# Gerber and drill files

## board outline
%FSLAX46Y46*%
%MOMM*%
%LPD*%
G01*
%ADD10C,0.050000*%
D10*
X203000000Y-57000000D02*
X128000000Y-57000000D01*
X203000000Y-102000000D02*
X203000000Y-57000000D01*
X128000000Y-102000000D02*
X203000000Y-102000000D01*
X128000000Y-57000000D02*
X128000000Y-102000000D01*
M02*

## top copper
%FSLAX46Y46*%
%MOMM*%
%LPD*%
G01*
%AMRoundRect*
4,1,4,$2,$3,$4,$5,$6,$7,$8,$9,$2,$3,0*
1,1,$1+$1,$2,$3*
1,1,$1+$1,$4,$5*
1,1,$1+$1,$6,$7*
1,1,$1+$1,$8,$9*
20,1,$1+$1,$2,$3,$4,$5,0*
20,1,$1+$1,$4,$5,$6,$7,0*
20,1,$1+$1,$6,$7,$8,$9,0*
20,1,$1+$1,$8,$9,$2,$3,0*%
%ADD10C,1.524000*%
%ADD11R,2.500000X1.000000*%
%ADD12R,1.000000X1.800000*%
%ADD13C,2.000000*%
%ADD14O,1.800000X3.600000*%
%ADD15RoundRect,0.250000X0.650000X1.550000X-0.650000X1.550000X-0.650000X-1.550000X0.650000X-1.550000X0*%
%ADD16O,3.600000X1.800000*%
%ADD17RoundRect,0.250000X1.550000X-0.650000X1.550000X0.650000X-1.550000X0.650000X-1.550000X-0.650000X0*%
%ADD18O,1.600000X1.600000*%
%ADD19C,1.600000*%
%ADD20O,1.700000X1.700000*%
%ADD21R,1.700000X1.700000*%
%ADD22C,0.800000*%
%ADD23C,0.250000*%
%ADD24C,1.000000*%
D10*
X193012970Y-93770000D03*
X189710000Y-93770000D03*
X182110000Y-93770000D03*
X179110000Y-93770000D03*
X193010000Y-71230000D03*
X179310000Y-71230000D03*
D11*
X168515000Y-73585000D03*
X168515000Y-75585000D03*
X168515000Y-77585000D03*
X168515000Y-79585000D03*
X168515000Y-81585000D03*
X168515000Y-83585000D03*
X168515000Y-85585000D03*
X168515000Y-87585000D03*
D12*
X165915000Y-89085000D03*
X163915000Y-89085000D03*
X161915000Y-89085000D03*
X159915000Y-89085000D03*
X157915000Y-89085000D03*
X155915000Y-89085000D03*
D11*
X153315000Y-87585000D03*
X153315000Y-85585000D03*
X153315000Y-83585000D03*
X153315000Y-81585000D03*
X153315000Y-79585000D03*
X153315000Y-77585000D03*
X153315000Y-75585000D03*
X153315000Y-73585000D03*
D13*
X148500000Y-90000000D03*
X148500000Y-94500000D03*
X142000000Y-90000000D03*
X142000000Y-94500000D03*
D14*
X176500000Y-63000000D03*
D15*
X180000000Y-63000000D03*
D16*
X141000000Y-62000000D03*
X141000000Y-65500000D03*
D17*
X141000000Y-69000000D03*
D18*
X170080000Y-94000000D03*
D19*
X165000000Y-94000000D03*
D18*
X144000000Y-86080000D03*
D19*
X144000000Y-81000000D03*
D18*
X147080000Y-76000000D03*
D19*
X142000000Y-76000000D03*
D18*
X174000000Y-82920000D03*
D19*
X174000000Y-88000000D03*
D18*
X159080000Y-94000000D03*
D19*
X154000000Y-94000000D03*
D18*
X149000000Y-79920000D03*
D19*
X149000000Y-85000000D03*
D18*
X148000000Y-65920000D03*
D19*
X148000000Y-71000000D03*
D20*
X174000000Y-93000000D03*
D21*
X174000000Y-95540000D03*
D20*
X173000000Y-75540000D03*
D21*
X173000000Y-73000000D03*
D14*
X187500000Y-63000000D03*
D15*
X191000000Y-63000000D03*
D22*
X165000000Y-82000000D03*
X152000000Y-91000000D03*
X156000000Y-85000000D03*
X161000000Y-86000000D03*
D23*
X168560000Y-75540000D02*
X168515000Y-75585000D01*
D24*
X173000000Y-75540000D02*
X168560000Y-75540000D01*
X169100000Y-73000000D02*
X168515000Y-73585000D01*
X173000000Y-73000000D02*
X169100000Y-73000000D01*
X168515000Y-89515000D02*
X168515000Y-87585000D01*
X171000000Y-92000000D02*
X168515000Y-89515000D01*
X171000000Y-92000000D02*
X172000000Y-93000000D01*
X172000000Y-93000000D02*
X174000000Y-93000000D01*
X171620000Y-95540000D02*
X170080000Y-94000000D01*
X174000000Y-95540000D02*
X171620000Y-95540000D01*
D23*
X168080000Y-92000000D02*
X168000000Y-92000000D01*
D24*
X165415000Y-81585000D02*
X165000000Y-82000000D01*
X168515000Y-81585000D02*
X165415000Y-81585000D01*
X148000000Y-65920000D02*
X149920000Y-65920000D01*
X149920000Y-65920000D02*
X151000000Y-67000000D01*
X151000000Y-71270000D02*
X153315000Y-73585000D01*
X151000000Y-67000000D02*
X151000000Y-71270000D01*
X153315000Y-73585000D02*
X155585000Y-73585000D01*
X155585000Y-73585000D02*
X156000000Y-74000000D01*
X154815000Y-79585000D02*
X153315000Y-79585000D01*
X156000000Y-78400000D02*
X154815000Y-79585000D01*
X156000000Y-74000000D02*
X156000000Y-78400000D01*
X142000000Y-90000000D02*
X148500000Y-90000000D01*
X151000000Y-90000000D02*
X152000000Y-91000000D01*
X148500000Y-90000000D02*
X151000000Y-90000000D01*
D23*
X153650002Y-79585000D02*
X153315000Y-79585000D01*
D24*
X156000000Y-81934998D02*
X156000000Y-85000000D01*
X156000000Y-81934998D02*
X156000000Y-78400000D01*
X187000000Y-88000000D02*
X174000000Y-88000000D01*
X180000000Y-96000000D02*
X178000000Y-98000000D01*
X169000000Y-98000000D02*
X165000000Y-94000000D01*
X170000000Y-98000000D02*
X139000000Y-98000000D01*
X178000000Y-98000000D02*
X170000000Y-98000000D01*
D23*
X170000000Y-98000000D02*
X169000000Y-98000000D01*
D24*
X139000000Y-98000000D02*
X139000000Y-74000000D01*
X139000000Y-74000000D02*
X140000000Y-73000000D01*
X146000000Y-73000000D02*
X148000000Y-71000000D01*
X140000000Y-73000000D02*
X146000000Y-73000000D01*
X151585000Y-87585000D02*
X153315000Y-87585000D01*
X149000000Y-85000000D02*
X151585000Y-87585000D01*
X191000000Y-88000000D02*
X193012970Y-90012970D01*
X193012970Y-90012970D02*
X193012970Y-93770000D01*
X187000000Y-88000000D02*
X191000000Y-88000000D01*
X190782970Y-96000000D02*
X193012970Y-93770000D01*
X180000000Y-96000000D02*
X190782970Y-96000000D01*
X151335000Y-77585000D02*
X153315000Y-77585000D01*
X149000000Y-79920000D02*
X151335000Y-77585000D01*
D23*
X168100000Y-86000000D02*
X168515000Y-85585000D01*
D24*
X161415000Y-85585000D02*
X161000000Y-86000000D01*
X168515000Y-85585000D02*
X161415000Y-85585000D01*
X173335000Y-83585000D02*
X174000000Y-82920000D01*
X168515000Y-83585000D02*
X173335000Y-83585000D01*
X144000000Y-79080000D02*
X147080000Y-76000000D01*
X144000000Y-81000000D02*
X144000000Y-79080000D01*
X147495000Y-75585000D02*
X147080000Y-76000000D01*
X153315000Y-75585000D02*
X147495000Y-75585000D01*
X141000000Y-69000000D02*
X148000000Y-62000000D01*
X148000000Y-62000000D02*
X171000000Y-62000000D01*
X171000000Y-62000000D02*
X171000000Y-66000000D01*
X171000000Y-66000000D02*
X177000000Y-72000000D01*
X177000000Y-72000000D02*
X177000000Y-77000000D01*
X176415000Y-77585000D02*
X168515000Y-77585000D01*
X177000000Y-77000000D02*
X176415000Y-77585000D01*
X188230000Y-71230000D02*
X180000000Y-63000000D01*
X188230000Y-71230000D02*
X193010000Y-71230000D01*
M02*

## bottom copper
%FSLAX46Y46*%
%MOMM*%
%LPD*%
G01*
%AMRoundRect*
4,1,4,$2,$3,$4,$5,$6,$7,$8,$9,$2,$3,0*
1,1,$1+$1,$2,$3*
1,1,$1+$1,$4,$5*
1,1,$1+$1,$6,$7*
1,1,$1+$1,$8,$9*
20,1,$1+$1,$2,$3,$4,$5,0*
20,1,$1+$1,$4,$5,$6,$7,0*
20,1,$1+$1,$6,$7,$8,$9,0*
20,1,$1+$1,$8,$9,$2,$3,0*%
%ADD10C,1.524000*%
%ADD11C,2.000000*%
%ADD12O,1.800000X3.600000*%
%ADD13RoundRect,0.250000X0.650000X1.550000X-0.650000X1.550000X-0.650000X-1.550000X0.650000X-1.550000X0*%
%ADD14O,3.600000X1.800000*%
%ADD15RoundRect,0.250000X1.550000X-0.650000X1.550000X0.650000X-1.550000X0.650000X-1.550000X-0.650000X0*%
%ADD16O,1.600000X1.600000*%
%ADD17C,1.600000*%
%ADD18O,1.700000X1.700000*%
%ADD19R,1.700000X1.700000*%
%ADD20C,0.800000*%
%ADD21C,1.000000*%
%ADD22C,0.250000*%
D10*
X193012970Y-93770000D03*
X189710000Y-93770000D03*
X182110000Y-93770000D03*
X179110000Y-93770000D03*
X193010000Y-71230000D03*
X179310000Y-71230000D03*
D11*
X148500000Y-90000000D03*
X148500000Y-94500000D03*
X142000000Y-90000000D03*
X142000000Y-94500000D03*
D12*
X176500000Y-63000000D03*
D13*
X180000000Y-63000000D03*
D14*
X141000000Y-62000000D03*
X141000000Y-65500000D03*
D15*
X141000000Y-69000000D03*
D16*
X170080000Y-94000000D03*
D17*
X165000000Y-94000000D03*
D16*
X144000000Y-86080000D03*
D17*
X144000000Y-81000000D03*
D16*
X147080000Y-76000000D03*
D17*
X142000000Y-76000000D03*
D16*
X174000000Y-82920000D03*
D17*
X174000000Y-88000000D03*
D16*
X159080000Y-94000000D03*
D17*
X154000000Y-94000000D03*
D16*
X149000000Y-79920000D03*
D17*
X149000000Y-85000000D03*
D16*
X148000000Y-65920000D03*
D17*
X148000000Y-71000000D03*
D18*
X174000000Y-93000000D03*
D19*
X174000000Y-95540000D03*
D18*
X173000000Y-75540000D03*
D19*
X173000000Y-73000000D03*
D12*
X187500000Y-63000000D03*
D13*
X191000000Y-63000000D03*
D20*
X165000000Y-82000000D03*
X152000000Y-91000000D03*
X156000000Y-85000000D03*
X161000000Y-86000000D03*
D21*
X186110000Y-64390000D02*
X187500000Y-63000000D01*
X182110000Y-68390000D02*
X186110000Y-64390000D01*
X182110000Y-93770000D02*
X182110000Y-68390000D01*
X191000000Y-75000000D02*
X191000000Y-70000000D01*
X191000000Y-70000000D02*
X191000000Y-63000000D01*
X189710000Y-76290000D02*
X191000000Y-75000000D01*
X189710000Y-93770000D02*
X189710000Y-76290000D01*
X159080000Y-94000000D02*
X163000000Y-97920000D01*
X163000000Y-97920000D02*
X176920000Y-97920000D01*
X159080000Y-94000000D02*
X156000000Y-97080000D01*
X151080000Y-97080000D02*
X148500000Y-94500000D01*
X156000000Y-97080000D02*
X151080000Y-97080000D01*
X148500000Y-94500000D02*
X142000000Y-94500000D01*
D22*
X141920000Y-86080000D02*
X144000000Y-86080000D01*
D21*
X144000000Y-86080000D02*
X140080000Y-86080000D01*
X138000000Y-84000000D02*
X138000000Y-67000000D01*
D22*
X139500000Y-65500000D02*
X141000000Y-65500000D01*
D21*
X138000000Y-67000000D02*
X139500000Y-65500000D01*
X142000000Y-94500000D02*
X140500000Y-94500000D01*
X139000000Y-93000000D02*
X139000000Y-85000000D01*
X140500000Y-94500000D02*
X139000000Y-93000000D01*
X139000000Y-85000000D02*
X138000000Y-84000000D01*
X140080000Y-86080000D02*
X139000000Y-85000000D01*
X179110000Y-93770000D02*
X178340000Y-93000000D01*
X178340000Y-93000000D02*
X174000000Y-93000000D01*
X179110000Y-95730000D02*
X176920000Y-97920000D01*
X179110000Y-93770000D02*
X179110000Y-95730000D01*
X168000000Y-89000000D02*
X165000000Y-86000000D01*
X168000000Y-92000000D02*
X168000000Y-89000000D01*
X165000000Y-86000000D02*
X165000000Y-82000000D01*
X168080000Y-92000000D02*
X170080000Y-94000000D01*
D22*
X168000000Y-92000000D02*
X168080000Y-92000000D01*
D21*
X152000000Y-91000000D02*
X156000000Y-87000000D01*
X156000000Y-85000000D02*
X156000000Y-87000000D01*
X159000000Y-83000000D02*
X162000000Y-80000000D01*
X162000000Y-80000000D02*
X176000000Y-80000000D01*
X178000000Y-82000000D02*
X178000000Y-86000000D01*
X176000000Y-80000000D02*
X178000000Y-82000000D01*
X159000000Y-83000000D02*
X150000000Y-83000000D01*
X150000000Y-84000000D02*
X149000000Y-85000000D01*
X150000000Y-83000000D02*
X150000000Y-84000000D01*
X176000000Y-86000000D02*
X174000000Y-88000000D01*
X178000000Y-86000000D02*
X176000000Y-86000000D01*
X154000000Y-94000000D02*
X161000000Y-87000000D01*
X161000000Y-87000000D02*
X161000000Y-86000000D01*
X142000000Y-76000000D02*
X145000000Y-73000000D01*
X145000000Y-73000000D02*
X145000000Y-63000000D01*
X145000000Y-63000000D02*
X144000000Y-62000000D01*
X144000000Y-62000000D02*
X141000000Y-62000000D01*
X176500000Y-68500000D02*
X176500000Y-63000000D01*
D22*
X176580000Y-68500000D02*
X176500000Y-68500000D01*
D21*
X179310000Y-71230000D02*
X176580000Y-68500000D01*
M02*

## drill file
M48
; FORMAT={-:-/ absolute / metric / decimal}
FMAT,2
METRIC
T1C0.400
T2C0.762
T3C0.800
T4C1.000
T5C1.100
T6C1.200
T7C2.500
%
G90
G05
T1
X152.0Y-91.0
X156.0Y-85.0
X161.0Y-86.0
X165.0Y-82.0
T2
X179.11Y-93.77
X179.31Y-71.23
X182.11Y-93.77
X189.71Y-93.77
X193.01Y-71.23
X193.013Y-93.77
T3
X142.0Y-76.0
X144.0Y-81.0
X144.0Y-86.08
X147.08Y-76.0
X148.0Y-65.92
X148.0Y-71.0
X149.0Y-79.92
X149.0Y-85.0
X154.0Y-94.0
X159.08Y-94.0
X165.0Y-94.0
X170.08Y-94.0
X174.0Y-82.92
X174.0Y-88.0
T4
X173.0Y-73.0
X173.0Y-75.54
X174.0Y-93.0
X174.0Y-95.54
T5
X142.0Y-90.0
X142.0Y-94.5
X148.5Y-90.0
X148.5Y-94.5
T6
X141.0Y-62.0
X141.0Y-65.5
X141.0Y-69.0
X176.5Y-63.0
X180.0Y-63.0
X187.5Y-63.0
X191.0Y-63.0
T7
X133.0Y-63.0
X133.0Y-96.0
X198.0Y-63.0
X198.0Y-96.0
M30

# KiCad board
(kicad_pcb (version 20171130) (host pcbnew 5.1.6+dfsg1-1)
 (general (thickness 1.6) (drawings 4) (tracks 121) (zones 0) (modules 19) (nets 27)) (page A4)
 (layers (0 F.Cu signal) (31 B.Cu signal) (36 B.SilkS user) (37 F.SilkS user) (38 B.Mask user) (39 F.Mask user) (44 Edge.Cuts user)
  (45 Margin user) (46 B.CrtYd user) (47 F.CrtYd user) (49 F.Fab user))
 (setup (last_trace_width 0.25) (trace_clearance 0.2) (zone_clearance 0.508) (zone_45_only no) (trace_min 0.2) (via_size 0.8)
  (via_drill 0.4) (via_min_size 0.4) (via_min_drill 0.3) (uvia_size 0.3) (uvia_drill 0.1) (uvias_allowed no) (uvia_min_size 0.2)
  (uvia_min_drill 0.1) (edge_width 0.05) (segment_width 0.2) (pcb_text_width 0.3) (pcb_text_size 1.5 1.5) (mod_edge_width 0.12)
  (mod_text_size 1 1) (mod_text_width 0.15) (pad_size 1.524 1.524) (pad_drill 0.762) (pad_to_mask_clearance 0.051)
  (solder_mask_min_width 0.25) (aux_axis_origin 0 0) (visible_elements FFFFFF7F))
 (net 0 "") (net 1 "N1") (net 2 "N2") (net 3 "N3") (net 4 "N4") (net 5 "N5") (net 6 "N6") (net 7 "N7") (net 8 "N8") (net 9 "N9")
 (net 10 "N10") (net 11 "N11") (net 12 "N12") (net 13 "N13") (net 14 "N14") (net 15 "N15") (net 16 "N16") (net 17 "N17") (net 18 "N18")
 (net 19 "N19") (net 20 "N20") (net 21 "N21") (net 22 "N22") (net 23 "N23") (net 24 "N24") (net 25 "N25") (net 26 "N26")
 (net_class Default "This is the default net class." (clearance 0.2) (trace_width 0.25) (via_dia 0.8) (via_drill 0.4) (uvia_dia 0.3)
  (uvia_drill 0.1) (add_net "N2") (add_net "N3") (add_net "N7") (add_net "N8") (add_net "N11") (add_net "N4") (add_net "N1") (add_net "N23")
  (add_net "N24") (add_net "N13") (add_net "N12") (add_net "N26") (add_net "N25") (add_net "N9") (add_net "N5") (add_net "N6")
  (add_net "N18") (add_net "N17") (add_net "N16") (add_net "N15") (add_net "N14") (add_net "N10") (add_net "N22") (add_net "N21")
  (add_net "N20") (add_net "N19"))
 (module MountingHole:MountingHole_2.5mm (layer F.Cu) (at 133 63)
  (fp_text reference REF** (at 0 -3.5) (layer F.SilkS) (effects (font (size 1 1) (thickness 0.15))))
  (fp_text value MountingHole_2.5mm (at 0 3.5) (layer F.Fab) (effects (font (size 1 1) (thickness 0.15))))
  (pad 1 np_thru_hole circle (at 0 0) (size 2.5 2.5) (drill 2.5) (layers *.Cu *.Mask)))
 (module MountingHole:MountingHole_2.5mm (layer F.Cu) (at 133 96)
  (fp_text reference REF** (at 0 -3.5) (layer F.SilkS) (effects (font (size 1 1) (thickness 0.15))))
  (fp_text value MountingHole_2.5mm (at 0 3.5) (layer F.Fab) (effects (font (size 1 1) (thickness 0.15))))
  (pad 1 np_thru_hole circle (at 0 0) (size 2.5 2.5) (drill 2.5) (layers *.Cu *.Mask)))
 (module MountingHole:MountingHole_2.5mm (layer F.Cu) (at 198 96)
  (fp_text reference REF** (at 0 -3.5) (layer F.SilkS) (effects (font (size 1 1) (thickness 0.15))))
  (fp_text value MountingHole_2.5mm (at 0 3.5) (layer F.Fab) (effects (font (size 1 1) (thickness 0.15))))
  (pad 1 np_thru_hole circle (at 0 0) (size 2.5 2.5) (drill 2.5) (layers *.Cu *.Mask)))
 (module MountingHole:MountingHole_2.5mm (layer F.Cu) (at 198 63)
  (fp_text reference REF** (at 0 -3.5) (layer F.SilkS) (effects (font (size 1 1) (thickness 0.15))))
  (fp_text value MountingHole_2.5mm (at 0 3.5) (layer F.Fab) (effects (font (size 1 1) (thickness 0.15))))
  (pad 1 np_thru_hole circle (at 0 0) (size 2.5 2.5) (drill 2.5) (layers *.Cu *.Mask)))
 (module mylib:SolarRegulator (layer F.Cu) (at 186 83)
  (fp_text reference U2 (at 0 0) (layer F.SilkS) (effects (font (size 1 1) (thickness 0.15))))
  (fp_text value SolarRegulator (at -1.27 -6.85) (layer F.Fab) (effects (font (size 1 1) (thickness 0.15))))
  (pad 6 thru_hole circle (at 7.01297 10.77) (size 1.524 1.524) (drill 0.762) (layers *.Cu *.Mask) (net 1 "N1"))
  (pad 5 thru_hole circle (at 3.71 10.77) (size 1.524 1.524) (drill 0.762) (layers *.Cu *.Mask) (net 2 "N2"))
  (pad 4 thru_hole circle (at -3.89 10.77) (size 1.524 1.524) (drill 0.762) (layers *.Cu *.Mask) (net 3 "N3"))
  (pad 3 thru_hole circle (at -6.89 10.77) (size 1.524 1.524) (drill 0.762) (layers *.Cu *.Mask) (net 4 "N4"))
  (pad 2 thru_hole circle (at 7.01 -11.77) (size 1.524 1.524) (drill 0.762) (layers *.Cu *.Mask) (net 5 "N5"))
  (pad 1 thru_hole circle (at -6.69 -11.77) (size 1.524 1.524) (drill 0.762) (layers *.Cu *.Mask) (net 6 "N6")))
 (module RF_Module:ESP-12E (layer F.Cu) (at 160.915 77.085)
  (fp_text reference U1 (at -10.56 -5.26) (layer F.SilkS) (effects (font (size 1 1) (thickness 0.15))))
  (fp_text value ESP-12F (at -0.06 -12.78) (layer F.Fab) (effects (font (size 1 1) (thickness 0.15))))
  (pad 22 smd rect (at 7.6 -3.5) (size 2.5 1) (layers F.Cu F.Paste F.Mask) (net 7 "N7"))
  (pad 21 smd rect (at 7.6 -1.5) (size 2.5 1) (layers F.Cu F.Paste F.Mask) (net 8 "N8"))
  (pad 20 smd rect (at 7.6 0.5) (size 2.5 1) (layers F.Cu F.Paste F.Mask) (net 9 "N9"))
  (pad 19 smd rect (at 7.6 2.5) (size 2.5 1) (layers F.Cu F.Paste F.Mask) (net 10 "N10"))
  (pad 18 smd rect (at 7.6 4.5) (size 2.5 1) (layers F.Cu F.Paste F.Mask) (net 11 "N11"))
  (pad 17 smd rect (at 7.6 6.5) (size 2.5 1) (layers F.Cu F.Paste F.Mask) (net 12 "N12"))
  (pad 16 smd rect (at 7.6 8.5) (size 2.5 1) (layers F.Cu F.Paste F.Mask) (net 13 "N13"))
  (pad 15 smd rect (at 7.6 10.5) (size 2.5 1) (layers F.Cu F.Paste F.Mask) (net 4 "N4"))
  (pad 14 smd rect (at 5 12) (size 1 1.8) (layers F.Cu F.Paste F.Mask) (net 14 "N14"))
  (pad 13 smd rect (at 3 12) (size 1 1.8) (layers F.Cu F.Paste F.Mask) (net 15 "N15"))
  (pad 12 smd rect (at 1 12) (size 1 1.8) (layers F.Cu F.Paste F.Mask) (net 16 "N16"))
  (pad 11 smd rect (at -1 12) (size 1 1.8) (layers F.Cu F.Paste F.Mask) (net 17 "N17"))
  (pad 10 smd rect (at -3 12) (size 1 1.8) (layers F.Cu F.Paste F.Mask) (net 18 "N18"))
  (pad 9 smd rect (at -5 12) (size 1 1.8) (layers F.Cu F.Paste F.Mask) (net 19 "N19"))
  (pad 8 smd rect (at -7.6 10.5) (size 2.5 1) (layers F.Cu F.Paste F.Mask) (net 1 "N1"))
  (pad 7 smd rect (at -7.6 8.5) (size 2.5 1) (layers F.Cu F.Paste F.Mask) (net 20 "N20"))
  (pad 6 smd rect (at -7.6 6.5) (size 2.5 1) (layers F.Cu F.Paste F.Mask) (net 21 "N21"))
  (pad 5 smd rect (at -7.6 4.5) (size 2.5 1) (layers F.Cu F.Paste F.Mask) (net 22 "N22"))
  (pad 4 smd rect (at -7.6 2.5) (size 2.5 1) (layers F.Cu F.Paste F.Mask) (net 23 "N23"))
  (pad 3 smd rect (at -7.6 0.5) (size 2.5 1) (layers F.Cu F.Paste F.Mask) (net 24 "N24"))
  (pad 2 smd rect (at -7.6 -1.5) (size 2.5 1) (layers F.Cu F.Paste F.Mask) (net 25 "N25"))
  (pad 1 smd rect (at -7.6 -3.5) (size 2.5 1) (layers F.Cu F.Paste F.Mask) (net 23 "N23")))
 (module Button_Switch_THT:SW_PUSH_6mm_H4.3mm (layer F.Cu) (at 142 90)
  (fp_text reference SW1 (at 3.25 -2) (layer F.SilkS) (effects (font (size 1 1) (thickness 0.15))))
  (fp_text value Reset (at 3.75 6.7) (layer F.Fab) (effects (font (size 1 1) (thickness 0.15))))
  (pad 1 thru_hole circle (at 6.5 0 90) (size 2 2) (drill 1.1) (layers *.Cu *.Mask) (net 23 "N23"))
  (pad 2 thru_hole circle (at 6.5 4.5 90) (size 2 2) (drill 1.1) (layers *.Cu *.Mask) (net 4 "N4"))
  (pad 1 thru_hole circle (at 0 0 90) (size 2 2) (drill 1.1) (layers *.Cu *.Mask) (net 23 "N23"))
  (pad 2 thru_hole circle (at 0 4.5 90) (size 2 2) (drill 1.1) (layers *.Cu *.Mask) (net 4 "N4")))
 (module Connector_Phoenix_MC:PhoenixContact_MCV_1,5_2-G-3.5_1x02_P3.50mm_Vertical (layer F.Cu) (at 180 63 180)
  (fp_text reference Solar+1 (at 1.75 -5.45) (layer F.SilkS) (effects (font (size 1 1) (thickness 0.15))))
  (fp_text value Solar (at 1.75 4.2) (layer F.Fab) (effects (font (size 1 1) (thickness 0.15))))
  (pad 2 thru_hole oval (at 3.5 0 180) (size 1.8 3.6) (drill 1.2) (layers *.Cu *.Mask) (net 6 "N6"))
  (pad 1 thru_hole roundrect (at 0 0 180) (size 1.8 3.6) (drill 1.2) (layers *.Cu *.Mask) (roundrect_rratio 0.138889) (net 5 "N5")))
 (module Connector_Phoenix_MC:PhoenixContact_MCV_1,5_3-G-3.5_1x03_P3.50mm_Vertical (layer F.Cu) (at 141 69 90)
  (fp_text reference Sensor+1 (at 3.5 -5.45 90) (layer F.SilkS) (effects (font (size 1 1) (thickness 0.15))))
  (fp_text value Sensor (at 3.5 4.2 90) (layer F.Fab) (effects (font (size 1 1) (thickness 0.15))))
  (pad 3 thru_hole oval (at 7 0 90) (size 1.8 3.6) (drill 1.2) (layers *.Cu *.Mask) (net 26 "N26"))
  (pad 2 thru_hole oval (at 3.5 0 90) (size 1.8 3.6) (drill 1.2) (layers *.Cu *.Mask) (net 4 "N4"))
  (pad 1 thru_hole roundrect (at 0 0 90) (size 1.8 3.6) (drill 1.2) (layers *.Cu *.Mask) (roundrect_rratio 0.138889) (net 9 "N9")))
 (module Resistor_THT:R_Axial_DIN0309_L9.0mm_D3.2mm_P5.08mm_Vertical (layer F.Cu) (at 165 94)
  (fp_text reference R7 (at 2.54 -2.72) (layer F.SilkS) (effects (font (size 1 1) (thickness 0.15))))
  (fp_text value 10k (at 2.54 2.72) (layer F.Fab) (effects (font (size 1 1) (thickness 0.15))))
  (pad 2 thru_hole oval (at 5.08 0) (size 1.6 1.6) (drill 0.8) (layers *.Cu *.Mask) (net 11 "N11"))
  (pad 1 thru_hole circle (at 0 0) (size 1.6 1.6) (drill 0.8) (layers *.Cu *.Mask) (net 1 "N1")))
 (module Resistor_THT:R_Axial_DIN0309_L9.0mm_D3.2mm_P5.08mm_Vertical (layer F.Cu) (at 144 81 270)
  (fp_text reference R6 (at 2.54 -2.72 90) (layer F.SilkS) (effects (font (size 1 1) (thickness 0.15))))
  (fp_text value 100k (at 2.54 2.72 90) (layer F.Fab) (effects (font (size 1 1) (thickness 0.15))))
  (pad 2 thru_hole oval (at 5.08 0 270) (size 1.6 1.6) (drill 0.8) (layers *.Cu *.Mask) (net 4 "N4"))
  (pad 1 thru_hole circle (at 0 0 270) (size 1.6 1.6) (drill 0.8) (layers *.Cu *.Mask) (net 25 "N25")))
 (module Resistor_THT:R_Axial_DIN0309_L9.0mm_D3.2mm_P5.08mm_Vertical (layer F.Cu) (at 142 76)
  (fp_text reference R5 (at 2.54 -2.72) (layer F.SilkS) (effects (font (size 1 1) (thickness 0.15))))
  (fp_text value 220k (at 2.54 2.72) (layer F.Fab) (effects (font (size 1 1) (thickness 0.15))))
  (pad 2 thru_hole oval (at 5.08 0) (size 1.6 1.6) (drill 0.8) (layers *.Cu *.Mask) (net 25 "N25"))
  (pad 1 thru_hole circle (at 0 0) (size 1.6 1.6) (drill 0.8) (layers *.Cu *.Mask) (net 26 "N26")))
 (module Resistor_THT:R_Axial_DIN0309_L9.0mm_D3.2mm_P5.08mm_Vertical (layer F.Cu) (at 174 88 90)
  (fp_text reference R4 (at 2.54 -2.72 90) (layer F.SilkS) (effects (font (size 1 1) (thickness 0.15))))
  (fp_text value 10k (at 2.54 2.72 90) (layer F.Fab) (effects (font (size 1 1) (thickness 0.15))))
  (pad 2 thru_hole oval (at 5.08 0 90) (size 1.6 1.6) (drill 0.8) (layers *.Cu *.Mask) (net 12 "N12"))
  (pad 1 thru_hole circle (at 0 0 90) (size 1.6 1.6) (drill 0.8) (layers *.Cu *.Mask) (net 1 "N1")))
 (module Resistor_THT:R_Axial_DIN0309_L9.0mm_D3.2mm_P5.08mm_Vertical (layer F.Cu) (at 154 94)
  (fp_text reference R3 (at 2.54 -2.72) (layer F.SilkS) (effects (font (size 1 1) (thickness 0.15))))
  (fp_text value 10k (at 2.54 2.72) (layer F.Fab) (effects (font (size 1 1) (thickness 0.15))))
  (pad 2 thru_hole oval (at 5.08 0) (size 1.6 1.6) (drill 0.8) (layers *.Cu *.Mask) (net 4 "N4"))
  (pad 1 thru_hole circle (at 0 0) (size 1.6 1.6) (drill 0.8) (layers *.Cu *.Mask) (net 13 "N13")))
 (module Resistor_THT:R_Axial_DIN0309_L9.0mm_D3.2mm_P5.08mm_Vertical (layer F.Cu) (at 149 85 90)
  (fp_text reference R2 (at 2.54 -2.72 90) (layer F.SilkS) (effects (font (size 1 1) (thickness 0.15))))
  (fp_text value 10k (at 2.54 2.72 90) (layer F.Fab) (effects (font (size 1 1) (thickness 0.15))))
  (pad 2 thru_hole oval (at 5.08 0 90) (size 1.6 1.6) (drill 0.8) (layers *.Cu *.Mask) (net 24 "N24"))
  (pad 1 thru_hole circle (at 0 0 90) (size 1.6 1.6) (drill 0.8) (layers *.Cu *.Mask) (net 1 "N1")))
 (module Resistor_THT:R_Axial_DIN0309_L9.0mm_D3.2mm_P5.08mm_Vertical (layer F.Cu) (at 148 71 90)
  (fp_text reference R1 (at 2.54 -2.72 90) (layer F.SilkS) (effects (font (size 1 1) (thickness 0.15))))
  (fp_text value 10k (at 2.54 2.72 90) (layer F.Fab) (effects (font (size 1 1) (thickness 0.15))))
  (pad 2 thru_hole oval (at 5.08 0 90) (size 1.6 1.6) (drill 0.8) (layers *.Cu *.Mask) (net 23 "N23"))
  (pad 1 thru_hole circle (at 0 0 90) (size 1.6 1.6) (drill 0.8) (layers *.Cu *.Mask) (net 1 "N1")))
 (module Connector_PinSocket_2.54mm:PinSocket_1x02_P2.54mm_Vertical (layer F.Cu) (at 174 95.54 180)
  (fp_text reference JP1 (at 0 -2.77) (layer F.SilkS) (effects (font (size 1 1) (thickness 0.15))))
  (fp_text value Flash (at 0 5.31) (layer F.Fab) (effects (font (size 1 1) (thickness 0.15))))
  (pad 2 thru_hole oval (at 0 2.54 180) (size 1.7 1.7) (drill 1) (layers *.Cu *.Mask) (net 4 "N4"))
  (pad 1 thru_hole rect (at 0 0 180) (size 1.7 1.7) (drill 1) (layers *.Cu *.Mask) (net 11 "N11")))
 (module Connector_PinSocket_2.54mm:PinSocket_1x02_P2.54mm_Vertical (layer F.Cu) (at 173 73)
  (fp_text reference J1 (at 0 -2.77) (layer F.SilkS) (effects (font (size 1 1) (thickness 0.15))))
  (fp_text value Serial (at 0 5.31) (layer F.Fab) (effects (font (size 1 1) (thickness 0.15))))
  (pad 2 thru_hole oval (at 0 2.54) (size 1.7 1.7) (drill 1) (layers *.Cu *.Mask) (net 8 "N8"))
  (pad 1 thru_hole rect (at 0 0) (size 1.7 1.7) (drill 1) (layers *.Cu *.Mask) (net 7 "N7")))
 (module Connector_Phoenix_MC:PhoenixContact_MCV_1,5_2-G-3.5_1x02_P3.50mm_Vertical (layer F.Cu) (at 191 63 180)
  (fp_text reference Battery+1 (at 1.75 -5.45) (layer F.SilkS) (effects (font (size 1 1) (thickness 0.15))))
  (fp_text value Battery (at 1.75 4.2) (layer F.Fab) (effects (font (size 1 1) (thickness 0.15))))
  (pad 2 thru_hole oval (at 3.5 0 180) (size 1.8 3.6) (drill 1.2) (layers *.Cu *.Mask) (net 3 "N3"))
  (pad 1 thru_hole roundrect (at 0 0 180) (size 1.8 3.6) (drill 1.2) (layers *.Cu *.Mask) (roundrect_rratio 0.138889) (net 2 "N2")))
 (gr_line (start 203 57) (end 128 57) (layer Edge.Cuts) (width 0.05))
 (gr_line (start 203 102) (end 203 57) (layer Edge.Cuts) (width 0.05))
 (gr_line (start 128 102) (end 203 102) (layer Edge.Cuts) (width 0.05))
 (gr_line (start 128 57) (end 128 102) (layer Edge.Cuts) (width 0.05))
 (segment (start 186.11 64.39) (end 187.5 63) (width 1) (layer B.Cu) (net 3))
 (segment (start 182.11 68.39) (end 186.11 64.39) (width 1) (layer B.Cu) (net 3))
 (segment (start 182.11 93.77) (end 182.11 68.39) (width 1) (layer B.Cu) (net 3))
 (segment (start 191 75) (end 191 70) (width 1) (layer B.Cu) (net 2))
 (segment (start 191 70) (end 191 63) (width 1) (layer B.Cu) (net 2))
 (segment (start 189.71 76.29) (end 191 75) (width 1) (layer B.Cu) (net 2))
 (segment (start 189.71 93.77) (end 189.71 76.29) (width 1) (layer B.Cu) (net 2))
 (segment (start 168.56 75.54) (end 168.515 75.585) (width 0.25) (layer F.Cu) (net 8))
 (segment (start 173 75.54) (end 168.56 75.54) (width 1) (layer F.Cu) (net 8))
 (segment (start 169.1 73) (end 168.515 73.585) (width 1) (layer F.Cu) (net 7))
 (segment (start 173 73) (end 169.1 73) (width 1) (layer F.Cu) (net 7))
 (segment (start 168.515 89.515) (end 168.515 87.585) (width 1) (layer F.Cu) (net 4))
 (segment (start 171 92) (end 168.515 89.515) (width 1) (layer F.Cu) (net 4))
 (segment (start 159.08 94) (end 163 97.92) (width 1) (layer B.Cu) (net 4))
 (segment (start 163 97.92) (end 176.92 97.92) (width 1) (layer B.Cu) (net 4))
 (segment (start 159.08 94) (end 156 97.08) (width 1) (layer B.Cu) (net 4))
 (segment (start 151.08 97.08) (end 148.5 94.5) (width 1) (layer B.Cu) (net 4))
 (segment (start 156 97.08) (end 151.08 97.08) (width 1) (layer B.Cu) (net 4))
 (segment (start 148.5 94.5) (end 142 94.5) (width 1) (layer B.Cu) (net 4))
 (segment (start 141.92 86.08) (end 144 86.08) (width 0.25) (layer B.Cu) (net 4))
 (segment (start 144 86.08) (end 140.08 86.08) (width 1) (layer B.Cu) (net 4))
 (segment (start 138 84) (end 138 67) (width 1) (layer B.Cu) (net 4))
 (segment (start 139.5 65.5) (end 141 65.5) (width 0.25) (layer B.Cu) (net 4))
 (segment (start 138 67) (end 139.5 65.5) (width 1) (layer B.Cu) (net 4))
 (segment (start 142 94.5) (end 140.5 94.5) (width 1) (layer B.Cu) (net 4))
 (segment (start 139 93) (end 139 85) (width 1) (layer B.Cu) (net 4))
 (segment (start 140.5 94.5) (end 139 93) (width 1) (layer B.Cu) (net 4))
 (segment (start 139 85) (end 138 84) (width 1) (layer B.Cu) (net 4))
 (segment (start 140.08 86.08) (end 139 85) (width 1) (layer B.Cu) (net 4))
 (segment (start 171 92) (end 172 93) (width 1) (layer F.Cu) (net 4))
 (segment (start 172 93) (end 174 93) (width 1) (layer F.Cu) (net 4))
 (segment (start 179.11 93.77) (end 178.34 93) (width 1) (layer B.Cu) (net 4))
 (segment (start 178.34 93) (end 174 93) (width 1) (layer B.Cu) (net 4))
 (segment (start 179.11 95.73) (end 176.92 97.92) (width 1) (layer B.Cu) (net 4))
 (segment (start 179.11 93.77) (end 179.11 95.73) (width 1) (layer B.Cu) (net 4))
 (segment (start 171.62 95.54) (end 170.08 94) (width 1) (layer F.Cu) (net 11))
 (segment (start 174 95.54) (end 171.62 95.54) (width 1) (layer F.Cu) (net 11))
 (segment (start 168.08 92) (end 168 92) (width 0.25) (layer F.Cu) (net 11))
 (segment (start 168 89) (end 165 86) (width 1) (layer B.Cu) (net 11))
 (segment (start 168 92) (end 168 89) (width 1) (layer B.Cu) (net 11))
 (via (at 165 82) (size 0.8) (drill 0.4) (layers F.Cu B.Cu) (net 11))
 (segment (start 165 86) (end 165 82) (width 1) (layer B.Cu) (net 11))
 (segment (start 165.415 81.585) (end 165 82) (width 1) (layer F.Cu) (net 11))
 (segment (start 168.515 81.585) (end 165.415 81.585) (width 1) (layer F.Cu) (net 11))
 (segment (start 168.08 92) (end 170.08 94) (width 1) (layer B.Cu) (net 11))
 (segment (start 168 92) (end 168.08 92) (width 0.25) (layer B.Cu) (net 11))
 (segment (start 148 65.92) (end 149.92 65.92) (width 1) (layer F.Cu) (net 23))
 (segment (start 149.92 65.92) (end 151 67) (width 1) (layer F.Cu) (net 23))
 (segment (start 151 71.27) (end 153.315 73.585) (width 1) (layer F.Cu) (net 23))
 (segment (start 151 67) (end 151 71.27) (width 1) (layer F.Cu) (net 23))
 (segment (start 153.315 73.585) (end 155.585 73.585) (width 1) (layer F.Cu) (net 23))
 (segment (start 155.585 73.585) (end 156 74) (width 1) (layer F.Cu) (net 23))
 (segment (start 154.815 79.585) (end 153.315 79.585) (width 1) (layer F.Cu) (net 23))
 (segment (start 156 78.4) (end 154.815 79.585) (width 1) (layer F.Cu) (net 23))
 (segment (start 156 74) (end 156 78.4) (width 1) (layer F.Cu) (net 23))
 (segment (start 142 90) (end 148.5 90) (width 1) (layer F.Cu) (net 23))
 (via (at 152 91) (size 0.8) (drill 0.4) (layers F.Cu B.Cu) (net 23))
 (segment (start 151 90) (end 152 91) (width 1) (layer F.Cu) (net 23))
 (segment (start 148.5 90) (end 151 90) (width 1) (layer F.Cu) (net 23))
 (segment (start 152 91) (end 156 87) (width 1) (layer B.Cu) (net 23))
 (segment (start 153.650002 79.585) (end 153.315 79.585) (width 0.25) (layer F.Cu) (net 23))
 (via (at 156 85) (size 0.8) (drill 0.4) (layers F.Cu B.Cu) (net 23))
 (segment (start 156 81.934998) (end 156 85) (width 1) (layer F.Cu) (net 23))
 (segment (start 156 85) (end 156 87) (width 1) (layer B.Cu) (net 23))
 (segment (start 156 81.934998) (end 156 78.4) (width 1) (layer F.Cu) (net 23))
 (segment (start 187 88) (end 174 88) (width 1) (layer F.Cu) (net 1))
 (segment (start 180 96) (end 178 98) (width 1) (layer F.Cu) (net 1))
 (segment (start 169 98) (end 165 94) (width 1) (layer F.Cu) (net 1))
 (segment (start 170 98) (end 139 98) (width 1) (layer F.Cu) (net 1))
 (segment (start 178 98) (end 170 98) (width 1) (layer F.Cu) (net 1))
 (segment (start 170 98) (end 169 98) (width 0.25) (layer F.Cu) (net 1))
 (segment (start 139 98) (end 139 74) (width 1) (layer F.Cu) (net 1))
 (segment (start 139 74) (end 140 73) (width 1) (layer F.Cu) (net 1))
 (segment (start 146 73) (end 148 71) (width 1) (layer F.Cu) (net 1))
 (segment (start 140 73) (end 146 73) (width 1) (layer F.Cu) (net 1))
 (segment (start 151.585 87.585) (end 153.315 87.585) (width 1) (layer F.Cu) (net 1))
 (segment (start 149 85) (end 151.585 87.585) (width 1) (layer F.Cu) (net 1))
 (segment (start 159 83) (end 162 80) (width 1) (layer B.Cu) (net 1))
 (segment (start 162 80) (end 176 80) (width 1) (layer B.Cu) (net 1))
 (segment (start 178 82) (end 178 86) (width 1) (layer B.Cu) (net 1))
 (segment (start 176 80) (end 178 82) (width 1) (layer B.Cu) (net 1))
 (segment (start 159 83) (end 150 83) (width 1) (layer B.Cu) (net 1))
 (segment (start 150 84) (end 149 85) (width 1) (layer B.Cu) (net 1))
 (segment (start 150 83) (end 150 84) (width 1) (layer B.Cu) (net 1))
 (segment (start 176 86) (end 174 88) (width 1) (layer B.Cu) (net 1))
 (segment (start 178 86) (end 176 86) (width 1) (layer B.Cu) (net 1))
 (segment (start 191 88) (end 193.01297 90.01297) (width 1) (layer F.Cu) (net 1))
 (segment (start 193.01297 90.01297) (end 193.01297 93.77) (width 1) (layer F.Cu) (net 1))
 (segment (start 187 88) (end 191 88) (width 1) (layer F.Cu) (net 1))
 (segment (start 190.78297 96) (end 193.01297 93.77) (width 1) (layer F.Cu) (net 1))
 (segment (start 180 96) (end 190.78297 96) (width 1) (layer F.Cu) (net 1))
 (segment (start 151.335 77.585) (end 153.315 77.585) (width 1) (layer F.Cu) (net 24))
 (segment (start 149 79.92) (end 151.335 77.585) (width 1) (layer F.Cu) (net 24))
 (segment (start 154 94) (end 161 87) (width 1) (layer B.Cu) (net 13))
 (via (at 161 86) (size 0.8) (drill 0.4) (layers F.Cu B.Cu) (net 13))
 (segment (start 161 87) (end 161 86) (width 1) (layer B.Cu) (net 13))
 (segment (start 168.1 86) (end 168.515 85.585) (width 0.25) (layer F.Cu) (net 13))
 (segment (start 161.415 85.585) (end 161 86) (width 1) (layer F.Cu) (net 13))
 (segment (start 168.515 85.585) (end 161.415 85.585) (width 1) (layer F.Cu) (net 13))
 (segment (start 173.335 83.585) (end 174 82.92) (width 1) (layer F.Cu) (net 12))
 (segment (start 168.515 83.585) (end 173.335 83.585) (width 1) (layer F.Cu) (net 12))
 (segment (start 144 79.08) (end 147.08 76) (width 1) (layer F.Cu) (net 25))
 (segment (start 144 81) (end 144 79.08) (width 1) (layer F.Cu) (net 25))
 (segment (start 147.495 75.585) (end 147.08 76) (width 1) (layer F.Cu) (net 25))
 (segment (start 153.315 75.585) (end 147.495 75.585) (width 1) (layer F.Cu) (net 25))
 (segment (start 142 76) (end 145 73) (width 1) (layer B.Cu) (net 26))
 (segment (start 145 73) (end 145 63) (width 1) (layer B.Cu) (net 26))
 (segment (start 145 63) (end 144 62) (width 1) (layer B.Cu) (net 26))
 (segment (start 144 62) (end 141 62) (width 1) (layer B.Cu) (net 26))
 (segment (start 141 69) (end 148 62) (width 1) (layer F.Cu) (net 9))
 (segment (start 148 62) (end 171 62) (width 1) (layer F.Cu) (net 9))
 (segment (start 171 62) (end 171 66) (width 1) (layer F.Cu) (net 9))
 (segment (start 171 66) (end 177 72) (width 1) (layer F.Cu) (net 9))
 (segment (start 177 72) (end 177 77) (width 1) (layer F.Cu) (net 9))
 (segment (start 176.415 77.585) (end 168.515 77.585) (width 1) (layer F.Cu) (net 9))
 (segment (start 177 77) (end 176.415 77.585) (width 1) (layer F.Cu) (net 9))
 (segment (start 176.5 68.5) (end 176.5 63) (width 1) (layer B.Cu) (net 6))
 (segment (start 176.58 68.5) (end 176.5 68.5) (width 0.25) (layer B.Cu) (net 6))
 (segment (start 179.31 71.23) (end 176.58 68.5) (width 1) (layer B.Cu) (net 6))
 (segment (start 188.23 71.23) (end 180 63) (width 1) (layer F.Cu) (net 5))
 (segment (start 188.23 71.23) (end 193.01 71.23) (width 1) (layer F.Cu) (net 5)))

